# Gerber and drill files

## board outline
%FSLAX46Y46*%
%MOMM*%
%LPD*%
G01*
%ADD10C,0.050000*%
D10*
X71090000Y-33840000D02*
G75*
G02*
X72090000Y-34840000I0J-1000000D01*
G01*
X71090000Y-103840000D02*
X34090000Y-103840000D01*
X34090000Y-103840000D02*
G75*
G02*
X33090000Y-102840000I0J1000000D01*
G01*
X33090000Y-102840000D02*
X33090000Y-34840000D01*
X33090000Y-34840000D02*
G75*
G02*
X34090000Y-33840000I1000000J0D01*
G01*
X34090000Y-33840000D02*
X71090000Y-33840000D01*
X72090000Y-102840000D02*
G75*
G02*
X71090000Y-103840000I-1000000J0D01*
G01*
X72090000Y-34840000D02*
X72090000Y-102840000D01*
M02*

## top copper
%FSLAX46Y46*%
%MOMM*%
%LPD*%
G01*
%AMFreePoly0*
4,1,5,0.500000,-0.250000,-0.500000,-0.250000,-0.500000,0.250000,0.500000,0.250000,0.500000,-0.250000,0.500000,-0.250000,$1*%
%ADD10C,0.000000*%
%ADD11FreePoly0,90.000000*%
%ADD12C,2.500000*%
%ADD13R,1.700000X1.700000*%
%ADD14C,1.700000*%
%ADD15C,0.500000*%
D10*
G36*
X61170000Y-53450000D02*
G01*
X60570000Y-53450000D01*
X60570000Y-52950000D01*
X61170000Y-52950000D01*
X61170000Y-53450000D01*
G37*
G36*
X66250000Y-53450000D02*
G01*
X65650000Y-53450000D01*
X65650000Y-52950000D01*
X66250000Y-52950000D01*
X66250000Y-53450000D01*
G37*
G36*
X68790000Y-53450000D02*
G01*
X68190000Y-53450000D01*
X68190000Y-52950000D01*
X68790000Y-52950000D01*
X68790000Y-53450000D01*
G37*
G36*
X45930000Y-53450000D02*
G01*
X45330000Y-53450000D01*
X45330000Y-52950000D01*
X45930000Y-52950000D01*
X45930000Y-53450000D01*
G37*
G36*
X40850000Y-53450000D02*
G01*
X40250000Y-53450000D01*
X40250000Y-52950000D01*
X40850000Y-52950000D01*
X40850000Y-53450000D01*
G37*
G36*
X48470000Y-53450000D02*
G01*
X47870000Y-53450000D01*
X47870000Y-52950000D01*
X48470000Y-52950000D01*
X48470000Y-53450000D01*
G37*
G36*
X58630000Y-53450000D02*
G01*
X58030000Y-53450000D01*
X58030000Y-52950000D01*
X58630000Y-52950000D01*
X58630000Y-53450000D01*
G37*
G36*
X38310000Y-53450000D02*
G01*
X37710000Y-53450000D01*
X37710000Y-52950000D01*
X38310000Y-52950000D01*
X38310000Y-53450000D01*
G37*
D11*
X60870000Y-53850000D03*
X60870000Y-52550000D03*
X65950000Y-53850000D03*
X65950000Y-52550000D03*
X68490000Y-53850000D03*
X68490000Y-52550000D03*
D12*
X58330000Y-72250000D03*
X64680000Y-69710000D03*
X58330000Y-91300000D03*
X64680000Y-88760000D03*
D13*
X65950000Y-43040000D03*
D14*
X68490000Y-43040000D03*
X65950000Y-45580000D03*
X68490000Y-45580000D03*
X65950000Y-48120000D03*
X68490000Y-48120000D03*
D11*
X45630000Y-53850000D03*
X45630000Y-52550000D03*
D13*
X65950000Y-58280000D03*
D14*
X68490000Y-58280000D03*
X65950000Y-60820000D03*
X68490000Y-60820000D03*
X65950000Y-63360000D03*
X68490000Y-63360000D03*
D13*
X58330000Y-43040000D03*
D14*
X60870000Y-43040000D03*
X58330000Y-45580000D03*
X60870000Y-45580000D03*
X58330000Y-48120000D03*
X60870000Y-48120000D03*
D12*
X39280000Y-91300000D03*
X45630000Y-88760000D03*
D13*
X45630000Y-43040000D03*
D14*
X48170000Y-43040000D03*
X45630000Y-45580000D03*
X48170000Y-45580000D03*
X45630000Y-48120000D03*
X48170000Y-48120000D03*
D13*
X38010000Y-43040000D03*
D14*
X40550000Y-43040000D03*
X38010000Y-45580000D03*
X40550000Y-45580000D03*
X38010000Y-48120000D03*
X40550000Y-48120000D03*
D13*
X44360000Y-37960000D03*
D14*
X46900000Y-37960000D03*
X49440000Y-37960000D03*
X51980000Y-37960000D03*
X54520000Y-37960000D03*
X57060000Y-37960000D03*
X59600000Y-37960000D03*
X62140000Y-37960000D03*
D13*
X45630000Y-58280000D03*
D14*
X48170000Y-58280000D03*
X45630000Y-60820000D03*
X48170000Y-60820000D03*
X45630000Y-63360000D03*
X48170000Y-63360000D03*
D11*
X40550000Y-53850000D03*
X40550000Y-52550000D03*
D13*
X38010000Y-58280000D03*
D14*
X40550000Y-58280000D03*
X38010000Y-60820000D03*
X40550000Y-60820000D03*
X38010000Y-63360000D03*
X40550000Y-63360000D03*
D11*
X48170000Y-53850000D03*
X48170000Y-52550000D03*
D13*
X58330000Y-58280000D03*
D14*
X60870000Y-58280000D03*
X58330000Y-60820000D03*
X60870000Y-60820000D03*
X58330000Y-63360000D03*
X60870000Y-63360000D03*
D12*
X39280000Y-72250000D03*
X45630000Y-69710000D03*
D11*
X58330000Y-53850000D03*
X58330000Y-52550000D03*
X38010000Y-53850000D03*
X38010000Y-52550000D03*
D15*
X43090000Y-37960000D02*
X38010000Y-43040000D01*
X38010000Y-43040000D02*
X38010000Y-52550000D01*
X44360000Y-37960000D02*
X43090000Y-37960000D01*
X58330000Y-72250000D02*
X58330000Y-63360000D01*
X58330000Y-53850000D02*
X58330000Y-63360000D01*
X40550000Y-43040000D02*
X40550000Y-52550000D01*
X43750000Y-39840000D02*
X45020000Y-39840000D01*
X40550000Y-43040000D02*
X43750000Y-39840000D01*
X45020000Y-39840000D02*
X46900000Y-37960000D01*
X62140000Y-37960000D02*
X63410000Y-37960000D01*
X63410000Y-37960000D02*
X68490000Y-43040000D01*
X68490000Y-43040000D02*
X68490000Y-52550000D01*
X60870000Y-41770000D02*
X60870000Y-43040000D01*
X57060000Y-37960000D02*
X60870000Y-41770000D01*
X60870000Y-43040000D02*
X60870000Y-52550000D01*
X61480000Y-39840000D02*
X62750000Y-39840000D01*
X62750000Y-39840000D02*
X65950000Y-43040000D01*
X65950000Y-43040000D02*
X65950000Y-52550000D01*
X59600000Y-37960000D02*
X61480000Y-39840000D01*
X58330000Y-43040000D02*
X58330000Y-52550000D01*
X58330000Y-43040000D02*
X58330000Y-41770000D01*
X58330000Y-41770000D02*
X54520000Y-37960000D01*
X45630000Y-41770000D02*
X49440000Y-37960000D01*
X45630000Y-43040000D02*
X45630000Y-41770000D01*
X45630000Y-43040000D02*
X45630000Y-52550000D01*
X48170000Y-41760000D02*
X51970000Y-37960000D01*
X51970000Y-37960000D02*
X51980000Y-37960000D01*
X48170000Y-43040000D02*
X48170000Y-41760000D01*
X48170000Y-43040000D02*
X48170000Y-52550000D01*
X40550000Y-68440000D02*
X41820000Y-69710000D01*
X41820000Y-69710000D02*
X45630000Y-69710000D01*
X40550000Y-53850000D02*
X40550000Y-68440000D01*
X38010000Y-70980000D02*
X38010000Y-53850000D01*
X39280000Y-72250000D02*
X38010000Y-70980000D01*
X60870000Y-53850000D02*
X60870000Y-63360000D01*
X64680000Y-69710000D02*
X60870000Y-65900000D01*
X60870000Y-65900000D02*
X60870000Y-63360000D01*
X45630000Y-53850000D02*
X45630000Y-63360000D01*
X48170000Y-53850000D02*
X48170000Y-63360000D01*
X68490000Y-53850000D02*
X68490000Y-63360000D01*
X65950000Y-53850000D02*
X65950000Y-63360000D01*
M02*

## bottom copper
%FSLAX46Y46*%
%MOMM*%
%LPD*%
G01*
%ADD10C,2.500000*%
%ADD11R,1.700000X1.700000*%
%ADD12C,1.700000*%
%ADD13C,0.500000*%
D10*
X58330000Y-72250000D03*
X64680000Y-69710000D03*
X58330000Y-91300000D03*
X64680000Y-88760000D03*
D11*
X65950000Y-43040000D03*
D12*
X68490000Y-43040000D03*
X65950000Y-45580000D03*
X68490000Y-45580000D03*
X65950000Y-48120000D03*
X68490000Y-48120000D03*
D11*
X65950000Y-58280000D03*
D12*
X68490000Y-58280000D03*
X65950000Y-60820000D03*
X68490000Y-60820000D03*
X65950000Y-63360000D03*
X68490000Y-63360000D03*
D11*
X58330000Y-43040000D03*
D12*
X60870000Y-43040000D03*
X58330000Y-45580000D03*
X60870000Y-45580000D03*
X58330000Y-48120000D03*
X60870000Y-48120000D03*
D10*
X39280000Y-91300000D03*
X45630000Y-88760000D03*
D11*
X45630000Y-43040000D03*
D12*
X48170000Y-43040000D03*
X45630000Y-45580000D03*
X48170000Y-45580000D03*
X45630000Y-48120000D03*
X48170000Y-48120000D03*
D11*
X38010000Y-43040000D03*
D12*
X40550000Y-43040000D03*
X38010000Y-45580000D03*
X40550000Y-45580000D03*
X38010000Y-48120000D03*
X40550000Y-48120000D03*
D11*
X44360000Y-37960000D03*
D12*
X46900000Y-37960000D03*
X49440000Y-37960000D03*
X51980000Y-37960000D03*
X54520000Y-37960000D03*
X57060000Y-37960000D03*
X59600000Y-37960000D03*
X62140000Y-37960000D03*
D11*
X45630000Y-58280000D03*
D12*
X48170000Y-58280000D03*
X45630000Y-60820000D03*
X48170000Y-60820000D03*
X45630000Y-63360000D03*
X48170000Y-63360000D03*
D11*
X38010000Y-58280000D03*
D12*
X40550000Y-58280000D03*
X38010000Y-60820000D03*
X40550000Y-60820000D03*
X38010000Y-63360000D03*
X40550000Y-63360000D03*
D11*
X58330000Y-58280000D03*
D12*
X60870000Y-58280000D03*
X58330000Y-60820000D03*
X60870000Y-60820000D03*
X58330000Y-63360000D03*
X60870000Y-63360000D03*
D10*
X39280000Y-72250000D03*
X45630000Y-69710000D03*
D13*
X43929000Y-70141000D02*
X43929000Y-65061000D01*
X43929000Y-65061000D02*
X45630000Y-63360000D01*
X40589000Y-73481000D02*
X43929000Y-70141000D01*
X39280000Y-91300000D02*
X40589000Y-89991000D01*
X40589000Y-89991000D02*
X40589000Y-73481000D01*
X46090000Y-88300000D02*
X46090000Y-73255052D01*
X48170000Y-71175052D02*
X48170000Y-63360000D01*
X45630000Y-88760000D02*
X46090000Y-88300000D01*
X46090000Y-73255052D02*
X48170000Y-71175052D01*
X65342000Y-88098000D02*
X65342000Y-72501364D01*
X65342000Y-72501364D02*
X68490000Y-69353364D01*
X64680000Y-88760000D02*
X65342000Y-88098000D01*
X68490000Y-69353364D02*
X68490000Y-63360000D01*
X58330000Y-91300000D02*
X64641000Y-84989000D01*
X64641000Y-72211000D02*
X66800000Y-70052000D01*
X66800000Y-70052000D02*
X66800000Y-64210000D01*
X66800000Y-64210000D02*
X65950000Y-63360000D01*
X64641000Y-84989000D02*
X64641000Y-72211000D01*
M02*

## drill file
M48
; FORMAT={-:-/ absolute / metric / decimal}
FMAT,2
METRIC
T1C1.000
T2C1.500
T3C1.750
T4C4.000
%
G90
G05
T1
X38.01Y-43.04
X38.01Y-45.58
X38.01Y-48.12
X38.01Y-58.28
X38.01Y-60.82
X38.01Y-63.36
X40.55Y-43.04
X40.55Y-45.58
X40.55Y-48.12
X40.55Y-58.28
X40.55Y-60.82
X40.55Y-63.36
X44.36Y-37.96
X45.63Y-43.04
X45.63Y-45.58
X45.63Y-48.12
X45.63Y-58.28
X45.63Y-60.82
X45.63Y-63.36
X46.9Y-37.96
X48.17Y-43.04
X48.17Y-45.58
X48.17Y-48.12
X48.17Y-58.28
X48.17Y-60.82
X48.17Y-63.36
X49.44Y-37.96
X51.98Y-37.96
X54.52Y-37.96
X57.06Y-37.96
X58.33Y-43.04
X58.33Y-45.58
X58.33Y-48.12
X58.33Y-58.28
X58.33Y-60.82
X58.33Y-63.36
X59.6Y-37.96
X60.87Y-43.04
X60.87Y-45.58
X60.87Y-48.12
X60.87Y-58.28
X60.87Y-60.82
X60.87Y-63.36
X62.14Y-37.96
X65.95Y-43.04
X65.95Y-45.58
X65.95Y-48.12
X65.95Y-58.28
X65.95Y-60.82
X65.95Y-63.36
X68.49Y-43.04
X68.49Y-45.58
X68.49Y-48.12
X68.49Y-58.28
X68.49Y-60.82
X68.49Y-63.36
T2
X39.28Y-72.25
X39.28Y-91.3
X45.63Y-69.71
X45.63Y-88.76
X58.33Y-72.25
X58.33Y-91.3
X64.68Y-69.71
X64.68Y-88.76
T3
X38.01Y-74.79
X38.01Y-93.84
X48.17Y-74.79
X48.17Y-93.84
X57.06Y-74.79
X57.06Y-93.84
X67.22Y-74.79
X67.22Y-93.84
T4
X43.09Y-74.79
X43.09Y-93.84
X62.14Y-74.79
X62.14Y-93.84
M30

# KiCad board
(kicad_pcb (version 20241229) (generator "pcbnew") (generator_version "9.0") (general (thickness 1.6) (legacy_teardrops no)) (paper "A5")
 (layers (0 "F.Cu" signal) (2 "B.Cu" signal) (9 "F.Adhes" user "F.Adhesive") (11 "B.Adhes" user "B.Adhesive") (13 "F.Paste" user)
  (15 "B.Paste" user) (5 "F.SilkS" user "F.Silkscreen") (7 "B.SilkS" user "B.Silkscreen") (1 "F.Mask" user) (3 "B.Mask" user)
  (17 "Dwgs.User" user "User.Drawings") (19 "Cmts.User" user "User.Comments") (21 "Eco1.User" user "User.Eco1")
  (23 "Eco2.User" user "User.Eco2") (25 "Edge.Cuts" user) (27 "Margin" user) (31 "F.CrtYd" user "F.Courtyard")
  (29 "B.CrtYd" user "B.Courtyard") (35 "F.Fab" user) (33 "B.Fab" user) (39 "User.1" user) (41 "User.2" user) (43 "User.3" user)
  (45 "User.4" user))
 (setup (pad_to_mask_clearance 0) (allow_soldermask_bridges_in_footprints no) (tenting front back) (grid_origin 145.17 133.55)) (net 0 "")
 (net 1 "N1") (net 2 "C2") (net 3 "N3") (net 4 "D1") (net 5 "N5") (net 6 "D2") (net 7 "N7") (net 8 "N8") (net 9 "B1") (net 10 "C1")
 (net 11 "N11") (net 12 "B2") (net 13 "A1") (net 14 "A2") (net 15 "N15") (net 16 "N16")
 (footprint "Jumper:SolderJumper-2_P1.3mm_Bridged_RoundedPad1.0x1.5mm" (layer "F.Cu") (at 60.87 53.2 90)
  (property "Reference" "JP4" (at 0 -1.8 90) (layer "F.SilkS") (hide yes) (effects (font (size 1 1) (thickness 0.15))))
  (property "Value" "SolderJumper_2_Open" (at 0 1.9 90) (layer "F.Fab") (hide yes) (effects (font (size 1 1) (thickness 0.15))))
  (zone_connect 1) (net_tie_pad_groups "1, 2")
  (fp_poly (pts (xy 0.25 -0.3) (xy -0.25 -0.3) (xy -0.25 0.3) (xy 0.25 0.3)) (stroke (width 0) (type solid)) (fill yes) (layer "F.Cu"))
  (pad "1" smd custom (at -0.65 0 90) (size 1 0.5) (layers "F.Cu" "F.Mask") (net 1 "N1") (zone_connect 2) (thermal_bridge_angle 45)
   (options (clearance outline) (anchor rect)) (primitives))
  (pad "2" smd custom (at 0.65 0 90) (size 1 0.5) (layers "F.Cu" "F.Mask") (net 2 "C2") (zone_connect 2) (thermal_bridge_angle 45)
   (options (clearance outline) (anchor rect)) (primitives)))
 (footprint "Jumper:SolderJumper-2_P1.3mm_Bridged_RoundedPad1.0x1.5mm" (layer "F.Cu") (at 65.95 53.2 90)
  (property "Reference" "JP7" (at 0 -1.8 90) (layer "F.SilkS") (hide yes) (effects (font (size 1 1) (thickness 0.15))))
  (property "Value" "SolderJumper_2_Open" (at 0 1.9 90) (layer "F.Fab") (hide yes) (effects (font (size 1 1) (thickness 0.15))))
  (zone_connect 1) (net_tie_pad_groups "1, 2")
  (fp_poly (pts (xy 0.25 -0.3) (xy -0.25 -0.3) (xy -0.25 0.3) (xy 0.25 0.3)) (stroke (width 0) (type solid)) (fill yes) (layer "F.Cu"))
  (pad "1" smd custom (at -0.65 0 90) (size 1 0.5) (layers "F.Cu" "F.Mask") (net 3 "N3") (zone_connect 2) (thermal_bridge_angle 45)
   (options (clearance outline) (anchor rect)) (primitives))
  (pad "2" smd custom (at 0.65 0 90) (size 1 0.5) (layers "F.Cu" "F.Mask") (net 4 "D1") (zone_connect 2) (thermal_bridge_angle 45)
   (options (clearance outline) (anchor rect)) (primitives)))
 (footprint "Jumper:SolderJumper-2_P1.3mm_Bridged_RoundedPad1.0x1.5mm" (layer "F.Cu") (at 68.49 53.2 90)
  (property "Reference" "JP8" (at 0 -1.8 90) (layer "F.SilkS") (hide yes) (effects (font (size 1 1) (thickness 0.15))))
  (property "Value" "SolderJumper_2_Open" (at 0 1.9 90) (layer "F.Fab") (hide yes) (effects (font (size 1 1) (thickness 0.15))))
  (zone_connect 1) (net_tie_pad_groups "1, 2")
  (fp_poly (pts (xy 0.25 -0.3) (xy -0.25 -0.3) (xy -0.25 0.3) (xy 0.25 0.3)) (stroke (width 0) (type solid)) (fill yes) (layer "F.Cu"))
  (pad "1" smd custom (at -0.65 0 90) (size 1 0.5) (layers "F.Cu" "F.Mask") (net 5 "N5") (zone_connect 2) (thermal_bridge_angle 45)
   (options (clearance outline) (anchor rect)) (primitives))
  (pad "2" smd custom (at 0.65 0 90) (size 1 0.5) (layers "F.Cu" "F.Mask") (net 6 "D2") (zone_connect 2) (thermal_bridge_angle 45)
   (options (clearance outline) (anchor rect)) (primitives)))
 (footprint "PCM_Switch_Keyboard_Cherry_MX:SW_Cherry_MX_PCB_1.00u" (layer "F.Cu") (at 62.14 74.79)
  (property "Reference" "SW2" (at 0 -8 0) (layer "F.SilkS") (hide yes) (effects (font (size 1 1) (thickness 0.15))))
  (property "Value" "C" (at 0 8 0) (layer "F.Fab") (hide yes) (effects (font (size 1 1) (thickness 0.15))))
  (pad "" np_thru_hole circle (at -5.08 0) (size 1.75 1.75) (drill 1.75) (layers "*.Cu" "*.Mask"))
  (pad "" np_thru_hole circle (at 0 0) (size 4 4) (drill 4) (layers "*.Cu" "*.Mask"))
  (pad "" np_thru_hole circle (at 5.08 0) (size 1.75 1.75) (drill 1.75) (layers "*.Cu" "*.Mask"))
  (pad "1" thru_hole circle (at -3.81 -2.54) (size 2.5 2.5) (drill 1.5) (layers "*.Cu" "*.Mask") (remove_unused_layers no) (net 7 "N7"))
  (pad "2" thru_hole circle (at 2.54 -5.08) (size 2.5 2.5) (drill 1.5) (layers "*.Cu" "*.Mask") (remove_unused_layers no) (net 1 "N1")))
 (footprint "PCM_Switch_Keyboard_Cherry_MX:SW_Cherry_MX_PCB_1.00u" (layer "F.Cu") (at 62.14 93.84)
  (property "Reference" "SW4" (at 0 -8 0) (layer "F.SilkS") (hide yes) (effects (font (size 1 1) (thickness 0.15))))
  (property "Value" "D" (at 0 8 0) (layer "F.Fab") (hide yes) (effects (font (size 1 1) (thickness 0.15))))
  (pad "" np_thru_hole circle (at -5.08 0) (size 1.75 1.75) (drill 1.75) (layers "*.Cu" "*.Mask"))
  (pad "" np_thru_hole circle (at 0 0) (size 4 4) (drill 4) (layers "*.Cu" "*.Mask"))
  (pad "" np_thru_hole circle (at 5.08 0) (size 1.75 1.75) (drill 1.75) (layers "*.Cu" "*.Mask"))
  (pad "1" thru_hole circle (at -3.81 -2.54) (size 2.5 2.5) (drill 1.5) (layers "*.Cu" "*.Mask") (remove_unused_layers no) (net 3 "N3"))
  (pad "2" thru_hole circle (at 2.54 -5.08) (size 2.5 2.5) (drill 1.5) (layers "*.Cu" "*.Mask") (remove_unused_layers no) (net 5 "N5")))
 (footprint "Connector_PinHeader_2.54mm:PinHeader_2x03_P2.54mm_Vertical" (layer "F.Cu") (at 65.95 43.04)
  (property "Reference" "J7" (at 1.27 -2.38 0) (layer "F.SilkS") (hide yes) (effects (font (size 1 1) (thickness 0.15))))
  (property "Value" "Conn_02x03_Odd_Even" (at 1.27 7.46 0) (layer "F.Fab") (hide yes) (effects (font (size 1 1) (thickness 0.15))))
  (pad "1" thru_hole rect (at 0 0) (size 1.7 1.7) (drill 1) (layers "*.Cu" "*.Mask") (remove_unused_layers no) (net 4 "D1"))
  (pad "2" thru_hole circle (at 2.54 0) (size 1.7 1.7) (drill 1) (layers "*.Cu" "*.Mask") (remove_unused_layers no) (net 6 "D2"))
  (pad "3" thru_hole circle (at 0 2.54) (size 1.7 1.7) (drill 1) (layers "*.Cu" "*.Mask") (remove_unused_layers no) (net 4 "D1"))
  (pad "4" thru_hole circle (at 2.54 2.54) (size 1.7 1.7) (drill 1) (layers "*.Cu" "*.Mask") (remove_unused_layers no) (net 6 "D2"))
  (pad "5" thru_hole circle (at 0 5.08) (size 1.7 1.7) (drill 1) (layers "*.Cu" "*.Mask") (remove_unused_layers no) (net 4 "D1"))
  (pad "6" thru_hole circle (at 2.54 5.08) (size 1.7 1.7) (drill 1) (layers "*.Cu" "*.Mask") (remove_unused_layers no) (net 6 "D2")))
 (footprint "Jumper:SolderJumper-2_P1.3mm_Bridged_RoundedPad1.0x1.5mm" (layer "F.Cu") (at 45.63 53.2 90)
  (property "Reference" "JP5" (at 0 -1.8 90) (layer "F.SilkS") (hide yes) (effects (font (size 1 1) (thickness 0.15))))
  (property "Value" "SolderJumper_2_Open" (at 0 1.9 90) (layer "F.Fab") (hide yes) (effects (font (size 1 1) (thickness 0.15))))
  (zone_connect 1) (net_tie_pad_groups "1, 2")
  (fp_poly (pts (xy 0.25 -0.3) (xy -0.25 -0.3) (xy -0.25 0.3) (xy 0.25 0.3)) (stroke (width 0) (type solid)) (fill yes) (layer "F.Cu"))
  (pad "1" smd custom (at -0.65 0 90) (size 1 0.5) (layers "F.Cu" "F.Mask") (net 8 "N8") (zone_connect 2) (thermal_bridge_angle 45)
   (options (clearance outline) (anchor rect)) (primitives))
  (pad "2" smd custom (at 0.65 0 90) (size 1 0.5) (layers "F.Cu" "F.Mask") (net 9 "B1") (zone_connect 2) (thermal_bridge_angle 45)
   (options (clearance outline) (anchor rect)) (primitives)))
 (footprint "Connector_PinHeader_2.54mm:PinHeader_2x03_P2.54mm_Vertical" (layer "F.Cu") (at 65.95 58.28)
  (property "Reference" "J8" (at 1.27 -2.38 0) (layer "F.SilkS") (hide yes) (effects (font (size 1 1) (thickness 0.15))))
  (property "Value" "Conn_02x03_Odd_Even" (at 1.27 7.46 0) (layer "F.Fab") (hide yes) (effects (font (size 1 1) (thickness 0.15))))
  (pad "1" thru_hole rect (at 0 0) (size 1.7 1.7) (drill 1) (layers "*.Cu" "*.Mask") (remove_unused_layers no) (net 3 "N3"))
  (pad "2" thru_hole circle (at 2.54 0) (size 1.7 1.7) (drill 1) (layers "*.Cu" "*.Mask") (remove_unused_layers no) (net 5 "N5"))
  (pad "3" thru_hole circle (at 0 2.54) (size 1.7 1.7) (drill 1) (layers "*.Cu" "*.Mask") (remove_unused_layers no) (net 3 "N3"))
  (pad "4" thru_hole circle (at 2.54 2.54) (size 1.7 1.7) (drill 1) (layers "*.Cu" "*.Mask") (remove_unused_layers no) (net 5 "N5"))
  (pad "5" thru_hole circle (at 0 5.08) (size 1.7 1.7) (drill 1) (layers "*.Cu" "*.Mask") (remove_unused_layers no) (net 3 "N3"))
  (pad "6" thru_hole circle (at 2.54 5.08) (size 1.7 1.7) (drill 1) (layers "*.Cu" "*.Mask") (remove_unused_layers no) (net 5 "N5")))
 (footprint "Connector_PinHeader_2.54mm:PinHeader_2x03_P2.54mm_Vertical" (layer "F.Cu") (at 58.33 43.04)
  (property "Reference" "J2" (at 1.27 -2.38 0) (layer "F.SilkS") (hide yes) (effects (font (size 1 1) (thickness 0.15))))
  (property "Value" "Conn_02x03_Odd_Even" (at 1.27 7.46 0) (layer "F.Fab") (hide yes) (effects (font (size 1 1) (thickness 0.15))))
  (pad "1" thru_hole rect (at 0 0) (size 1.7 1.7) (drill 1) (layers "*.Cu" "*.Mask") (remove_unused_layers no) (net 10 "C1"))
  (pad "2" thru_hole circle (at 2.54 0) (size 1.7 1.7) (drill 1) (layers "*.Cu" "*.Mask") (remove_unused_layers no) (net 2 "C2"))
  (pad "3" thru_hole circle (at 0 2.54) (size 1.7 1.7) (drill 1) (layers "*.Cu" "*.Mask") (remove_unused_layers no) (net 10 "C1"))
  (pad "4" thru_hole circle (at 2.54 2.54) (size 1.7 1.7) (drill 1) (layers "*.Cu" "*.Mask") (remove_unused_layers no) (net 2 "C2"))
  (pad "5" thru_hole circle (at 0 5.08) (size 1.7 1.7) (drill 1) (layers "*.Cu" "*.Mask") (remove_unused_layers no) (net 10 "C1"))
  (pad "6" thru_hole circle (at 2.54 5.08) (size 1.7 1.7) (drill 1) (layers "*.Cu" "*.Mask") (remove_unused_layers no) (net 2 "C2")))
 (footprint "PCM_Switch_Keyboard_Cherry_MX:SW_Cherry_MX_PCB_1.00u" (layer "F.Cu") (at 43.09 93.84)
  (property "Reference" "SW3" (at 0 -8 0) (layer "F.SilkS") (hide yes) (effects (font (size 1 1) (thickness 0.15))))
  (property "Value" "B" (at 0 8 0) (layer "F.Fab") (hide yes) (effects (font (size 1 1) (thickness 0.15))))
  (pad "" np_thru_hole circle (at -5.08 0) (size 1.75 1.75) (drill 1.75) (layers "*.Cu" "*.Mask"))
  (pad "" np_thru_hole circle (at 0 0) (size 4 4) (drill 4) (layers "*.Cu" "*.Mask"))
  (pad "" np_thru_hole circle (at 5.08 0) (size 1.75 1.75) (drill 1.75) (layers "*.Cu" "*.Mask"))
  (pad "1" thru_hole circle (at -3.81 -2.54) (size 2.5 2.5) (drill 1.5) (layers "*.Cu" "*.Mask") (remove_unused_layers no) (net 8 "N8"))
  (pad "2" thru_hole circle (at 2.54 -5.08) (size 2.5 2.5) (drill 1.5) (layers "*.Cu" "*.Mask") (remove_unused_layers no) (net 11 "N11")))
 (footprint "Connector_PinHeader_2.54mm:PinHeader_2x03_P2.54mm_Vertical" (layer "F.Cu") (at 45.63 43.04)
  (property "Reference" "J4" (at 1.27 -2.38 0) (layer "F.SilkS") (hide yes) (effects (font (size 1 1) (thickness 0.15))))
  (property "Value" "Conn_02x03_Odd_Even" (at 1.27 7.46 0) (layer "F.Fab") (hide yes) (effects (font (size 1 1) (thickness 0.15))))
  (pad "1" thru_hole rect (at 0 0) (size 1.7 1.7) (drill 1) (layers "*.Cu" "*.Mask") (remove_unused_layers no) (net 9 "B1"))
  (pad "2" thru_hole circle (at 2.54 0) (size 1.7 1.7) (drill 1) (layers "*.Cu" "*.Mask") (remove_unused_layers no) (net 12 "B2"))
  (pad "3" thru_hole circle (at 0 2.54) (size 1.7 1.7) (drill 1) (layers "*.Cu" "*.Mask") (remove_unused_layers no) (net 9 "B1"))
  (pad "4" thru_hole circle (at 2.54 2.54) (size 1.7 1.7) (drill 1) (layers "*.Cu" "*.Mask") (remove_unused_layers no) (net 12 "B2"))
  (pad "5" thru_hole circle (at 0 5.08) (size 1.7 1.7) (drill 1) (layers "*.Cu" "*.Mask") (remove_unused_layers no) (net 9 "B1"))
  (pad "6" thru_hole circle (at 2.54 5.08) (size 1.7 1.7) (drill 1) (layers "*.Cu" "*.Mask") (remove_unused_layers no) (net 12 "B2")))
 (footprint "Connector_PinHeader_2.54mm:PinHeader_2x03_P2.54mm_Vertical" (layer "F.Cu") (at 38.01 43.04)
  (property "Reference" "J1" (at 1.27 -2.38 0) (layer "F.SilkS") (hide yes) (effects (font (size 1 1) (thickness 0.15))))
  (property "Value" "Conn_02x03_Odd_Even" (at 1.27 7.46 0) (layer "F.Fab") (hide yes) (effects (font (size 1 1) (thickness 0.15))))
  (pad "1" thru_hole rect (at 0 0) (size 1.7 1.7) (drill 1) (layers "*.Cu" "*.Mask") (remove_unused_layers no) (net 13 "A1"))
  (pad "2" thru_hole circle (at 2.54 0) (size 1.7 1.7) (drill 1) (layers "*.Cu" "*.Mask") (remove_unused_layers no) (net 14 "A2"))
  (pad "3" thru_hole circle (at 0 2.54) (size 1.7 1.7) (drill 1) (layers "*.Cu" "*.Mask") (remove_unused_layers no) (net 13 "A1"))
  (pad "4" thru_hole circle (at 2.54 2.54) (size 1.7 1.7) (drill 1) (layers "*.Cu" "*.Mask") (remove_unused_layers no) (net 14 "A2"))
  (pad "5" thru_hole circle (at 0 5.08) (size 1.7 1.7) (drill 1) (layers "*.Cu" "*.Mask") (remove_unused_layers no) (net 13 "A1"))
  (pad "6" thru_hole circle (at 2.54 5.08) (size 1.7 1.7) (drill 1) (layers "*.Cu" "*.Mask") (remove_unused_layers no) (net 14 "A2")))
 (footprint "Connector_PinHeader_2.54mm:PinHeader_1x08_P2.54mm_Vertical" (layer "F.Cu") (at 44.36 37.96 90)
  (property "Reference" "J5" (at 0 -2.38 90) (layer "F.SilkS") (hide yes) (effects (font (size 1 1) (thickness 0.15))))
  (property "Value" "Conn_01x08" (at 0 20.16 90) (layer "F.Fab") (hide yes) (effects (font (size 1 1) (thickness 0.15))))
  (pad "1" thru_hole rect (at 0 0 90) (size 1.7 1.7) (drill 1) (layers "*.Cu" "*.Mask") (remove_unused_layers no) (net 13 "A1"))
  (pad "2" thru_hole circle (at 0 2.54 90) (size 1.7 1.7) (drill 1) (layers "*.Cu" "*.Mask") (remove_unused_layers no) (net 14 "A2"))
  (pad "3" thru_hole circle (at 0 5.08 90) (size 1.7 1.7) (drill 1) (layers "*.Cu" "*.Mask") (remove_unused_layers no) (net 9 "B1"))
  (pad "4" thru_hole circle (at 0 7.62 90) (size 1.7 1.7) (drill 1) (layers "*.Cu" "*.Mask") (remove_unused_layers no) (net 12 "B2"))
  (pad "5" thru_hole circle (at 0 10.16 90) (size 1.7 1.7) (drill 1) (layers "*.Cu" "*.Mask") (remove_unused_layers no) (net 10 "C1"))
  (pad "6" thru_hole circle (at 0 12.7 90) (size 1.7 1.7) (drill 1) (layers "*.Cu" "*.Mask") (remove_unused_layers no) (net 2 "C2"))
  (pad "7" thru_hole circle (at 0 15.24 90) (size 1.7 1.7) (drill 1) (layers "*.Cu" "*.Mask") (remove_unused_layers no) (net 4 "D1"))
  (pad "8" thru_hole circle (at 0 17.78 90) (size 1.7 1.7) (drill 1) (layers "*.Cu" "*.Mask") (remove_unused_layers no) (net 6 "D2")))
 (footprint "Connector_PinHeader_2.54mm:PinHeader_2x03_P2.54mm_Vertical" (layer "F.Cu") (at 45.63 58.28)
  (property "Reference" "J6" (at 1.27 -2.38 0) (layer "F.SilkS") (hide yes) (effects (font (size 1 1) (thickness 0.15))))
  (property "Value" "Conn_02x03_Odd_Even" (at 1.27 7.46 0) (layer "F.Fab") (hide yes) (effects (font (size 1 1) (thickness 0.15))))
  (pad "1" thru_hole rect (at 0 0) (size 1.7 1.7) (drill 1) (layers "*.Cu" "*.Mask") (remove_unused_layers no) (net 8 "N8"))
  (pad "2" thru_hole circle (at 2.54 0) (size 1.7 1.7) (drill 1) (layers "*.Cu" "*.Mask") (remove_unused_layers no) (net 11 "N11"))
  (pad "3" thru_hole circle (at 0 2.54) (size 1.7 1.7) (drill 1) (layers "*.Cu" "*.Mask") (remove_unused_layers no) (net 8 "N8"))
  (pad "4" thru_hole circle (at 2.54 2.54) (size 1.7 1.7) (drill 1) (layers "*.Cu" "*.Mask") (remove_unused_layers no) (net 11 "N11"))
  (pad "5" thru_hole circle (at 0 5.08) (size 1.7 1.7) (drill 1) (layers "*.Cu" "*.Mask") (remove_unused_layers no) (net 8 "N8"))
  (pad "6" thru_hole circle (at 2.54 5.08) (size 1.7 1.7) (drill 1) (layers "*.Cu" "*.Mask") (remove_unused_layers no) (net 11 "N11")))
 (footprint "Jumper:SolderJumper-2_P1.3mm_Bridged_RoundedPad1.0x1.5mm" (layer "F.Cu") (at 40.55 53.2 90)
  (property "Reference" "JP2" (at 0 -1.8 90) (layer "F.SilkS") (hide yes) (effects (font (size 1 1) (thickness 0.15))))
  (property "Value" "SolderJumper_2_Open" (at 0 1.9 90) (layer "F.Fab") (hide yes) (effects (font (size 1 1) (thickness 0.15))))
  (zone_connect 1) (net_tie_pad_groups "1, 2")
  (fp_poly (pts (xy 0.25 -0.3) (xy -0.25 -0.3) (xy -0.25 0.3) (xy 0.25 0.3)) (stroke (width 0) (type solid)) (fill yes) (layer "F.Cu"))
  (pad "1" smd custom (at -0.65 0 90) (size 1 0.5) (layers "F.Cu" "F.Mask") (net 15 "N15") (zone_connect 2) (thermal_bridge_angle 45)
   (options (clearance outline) (anchor rect)) (primitives))
  (pad "2" smd custom (at 0.65 0 90) (size 1 0.5) (layers "F.Cu" "F.Mask") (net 14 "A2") (zone_connect 2) (thermal_bridge_angle 45)
   (options (clearance outline) (anchor rect)) (primitives)))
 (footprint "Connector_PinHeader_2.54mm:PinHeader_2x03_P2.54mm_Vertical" (layer "F.Cu") (at 38.01 58.28)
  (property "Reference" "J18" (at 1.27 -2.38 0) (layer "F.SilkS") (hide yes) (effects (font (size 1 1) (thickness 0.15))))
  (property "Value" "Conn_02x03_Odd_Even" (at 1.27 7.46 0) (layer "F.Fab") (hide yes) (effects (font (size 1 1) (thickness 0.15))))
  (pad "1" thru_hole rect (at 0 0) (size 1.7 1.7) (drill 1) (layers "*.Cu" "*.Mask") (remove_unused_layers no) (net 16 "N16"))
  (pad "2" thru_hole circle (at 2.54 0) (size 1.7 1.7) (drill 1) (layers "*.Cu" "*.Mask") (remove_unused_layers no) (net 15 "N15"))
  (pad "3" thru_hole circle (at 0 2.54) (size 1.7 1.7) (drill 1) (layers "*.Cu" "*.Mask") (remove_unused_layers no) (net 16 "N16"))
  (pad "4" thru_hole circle (at 2.54 2.54) (size 1.7 1.7) (drill 1) (layers "*.Cu" "*.Mask") (remove_unused_layers no) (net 15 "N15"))
  (pad "5" thru_hole circle (at 0 5.08) (size 1.7 1.7) (drill 1) (layers "*.Cu" "*.Mask") (remove_unused_layers no) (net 16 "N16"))
  (pad "6" thru_hole circle (at 2.54 5.08) (size 1.7 1.7) (drill 1) (layers "*.Cu" "*.Mask") (remove_unused_layers no) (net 15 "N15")))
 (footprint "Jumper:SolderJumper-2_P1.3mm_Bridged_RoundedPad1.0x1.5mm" (layer "F.Cu") (at 48.17 53.2 90)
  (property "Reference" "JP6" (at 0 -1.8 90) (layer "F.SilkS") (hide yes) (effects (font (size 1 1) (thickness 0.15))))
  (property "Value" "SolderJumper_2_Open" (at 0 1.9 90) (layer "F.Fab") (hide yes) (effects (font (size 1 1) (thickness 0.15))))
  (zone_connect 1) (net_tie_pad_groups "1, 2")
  (fp_poly (pts (xy 0.25 -0.3) (xy -0.25 -0.3) (xy -0.25 0.3) (xy 0.25 0.3)) (stroke (width 0) (type solid)) (fill yes) (layer "F.Cu"))
  (pad "1" smd custom (at -0.65 0 90) (size 1 0.5) (layers "F.Cu" "F.Mask") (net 11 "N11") (zone_connect 2) (thermal_bridge_angle 45)
   (options (clearance outline) (anchor rect)) (primitives))
  (pad "2" smd custom (at 0.65 0 90) (size 1 0.5) (layers "F.Cu" "F.Mask") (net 12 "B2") (zone_connect 2) (thermal_bridge_angle 45)
   (options (clearance outline) (anchor rect)) (primitives)))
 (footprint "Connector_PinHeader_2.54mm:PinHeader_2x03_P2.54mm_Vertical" (layer "F.Cu") (at 58.33 58.28)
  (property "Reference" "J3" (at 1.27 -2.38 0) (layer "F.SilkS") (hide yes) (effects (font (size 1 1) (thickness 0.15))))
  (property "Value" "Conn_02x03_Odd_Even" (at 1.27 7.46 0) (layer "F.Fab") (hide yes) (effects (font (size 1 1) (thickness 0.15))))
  (pad "1" thru_hole rect (at 0 0) (size 1.7 1.7) (drill 1) (layers "*.Cu" "*.Mask") (remove_unused_layers no) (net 7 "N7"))
  (pad "2" thru_hole circle (at 2.54 0) (size 1.7 1.7) (drill 1) (layers "*.Cu" "*.Mask") (remove_unused_layers no) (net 1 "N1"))
  (pad "3" thru_hole circle (at 0 2.54) (size 1.7 1.7) (drill 1) (layers "*.Cu" "*.Mask") (remove_unused_layers no) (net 7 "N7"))
  (pad "4" thru_hole circle (at 2.54 2.54) (size 1.7 1.7) (drill 1) (layers "*.Cu" "*.Mask") (remove_unused_layers no) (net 1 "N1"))
  (pad "5" thru_hole circle (at 0 5.08) (size 1.7 1.7) (drill 1) (layers "*.Cu" "*.Mask") (remove_unused_layers no) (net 7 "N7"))
  (pad "6" thru_hole circle (at 2.54 5.08) (size 1.7 1.7) (drill 1) (layers "*.Cu" "*.Mask") (remove_unused_layers no) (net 1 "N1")))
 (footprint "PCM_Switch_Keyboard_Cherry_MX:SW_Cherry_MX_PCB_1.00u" (layer "F.Cu") (at 43.09 74.79)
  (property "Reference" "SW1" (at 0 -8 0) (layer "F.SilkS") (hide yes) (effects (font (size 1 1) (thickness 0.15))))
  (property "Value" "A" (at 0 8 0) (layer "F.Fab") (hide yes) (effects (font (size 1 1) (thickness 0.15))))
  (pad "" np_thru_hole circle (at -5.08 0) (size 1.75 1.75) (drill 1.75) (layers "*.Cu" "*.Mask"))
  (pad "" np_thru_hole circle (at 0 0) (size 4 4) (drill 4) (layers "*.Cu" "*.Mask"))
  (pad "" np_thru_hole circle (at 5.08 0) (size 1.75 1.75) (drill 1.75) (layers "*.Cu" "*.Mask"))
  (pad "1" thru_hole circle (at -3.81 -2.54) (size 2.5 2.5) (drill 1.5) (layers "*.Cu" "*.Mask") (remove_unused_layers no) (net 16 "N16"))
  (pad "2" thru_hole circle (at 2.54 -5.08) (size 2.5 2.5) (drill 1.5) (layers "*.Cu" "*.Mask") (remove_unused_layers no) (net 15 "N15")))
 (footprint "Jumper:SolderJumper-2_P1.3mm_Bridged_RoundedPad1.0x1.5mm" (layer "F.Cu") (at 58.33 53.2 90)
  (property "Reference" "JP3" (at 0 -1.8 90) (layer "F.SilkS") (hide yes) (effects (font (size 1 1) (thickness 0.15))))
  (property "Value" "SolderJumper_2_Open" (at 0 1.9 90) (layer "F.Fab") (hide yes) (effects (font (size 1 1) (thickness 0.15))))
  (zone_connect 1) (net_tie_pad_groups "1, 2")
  (fp_poly (pts (xy 0.25 -0.3) (xy -0.25 -0.3) (xy -0.25 0.3) (xy 0.25 0.3)) (stroke (width 0) (type solid)) (fill yes) (layer "F.Cu"))
  (pad "1" smd custom (at -0.65 0 90) (size 1 0.5) (layers "F.Cu" "F.Mask") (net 7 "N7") (zone_connect 2) (thermal_bridge_angle 45)
   (options (clearance outline) (anchor rect)) (primitives))
  (pad "2" smd custom (at 0.65 0 90) (size 1 0.5) (layers "F.Cu" "F.Mask") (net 10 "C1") (zone_connect 2) (thermal_bridge_angle 45)
   (options (clearance outline) (anchor rect)) (primitives)))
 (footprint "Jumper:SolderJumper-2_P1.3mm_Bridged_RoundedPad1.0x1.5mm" (layer "F.Cu") (at 38.01 53.2 90)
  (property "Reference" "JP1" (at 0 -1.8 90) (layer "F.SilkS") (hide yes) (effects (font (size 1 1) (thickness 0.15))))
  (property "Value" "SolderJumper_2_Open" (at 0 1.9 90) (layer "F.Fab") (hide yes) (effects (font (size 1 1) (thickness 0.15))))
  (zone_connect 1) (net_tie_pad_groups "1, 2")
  (fp_poly (pts (xy 0.25 -0.3) (xy -0.25 -0.3) (xy -0.25 0.3) (xy 0.25 0.3)) (stroke (width 0) (type solid)) (fill yes) (layer "F.Cu"))
  (pad "1" smd custom (at -0.65 0 90) (size 1 0.5) (layers "F.Cu" "F.Mask") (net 16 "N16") (zone_connect 2) (thermal_bridge_angle 45)
   (options (clearance outline) (anchor rect)) (primitives))
  (pad "2" smd custom (at 0.65 0 90) (size 1 0.5) (layers "F.Cu" "F.Mask") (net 13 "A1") (zone_connect 2) (thermal_bridge_angle 45)
   (options (clearance outline) (anchor rect)) (primitives)))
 (gr_arc (start 71.09 33.84) (mid 71.797107 34.132893) (end 72.09 34.84) (stroke (width 0.05) (type default)) (layer "Edge.Cuts"))
 (gr_line (start 71.09 103.84) (end 34.09 103.84) (stroke (width 0.05) (type default)) (layer "Edge.Cuts"))
 (gr_arc (start 34.09 103.84) (mid 33.382893 103.547107) (end 33.09 102.84) (stroke (width 0.05) (type default)) (layer "Edge.Cuts"))
 (gr_line (start 33.09 102.84) (end 33.09 34.84) (stroke (width 0.05) (type default)) (layer "Edge.Cuts"))
 (gr_arc (start 33.09 34.84) (mid 33.382893 34.132893) (end 34.09 33.84) (stroke (width 0.05) (type default)) (layer "Edge.Cuts"))
 (gr_line (start 34.09 33.84) (end 71.09 33.84) (stroke (width 0.05) (type default)) (layer "Edge.Cuts"))
 (gr_arc (start 72.09 102.84) (mid 71.797107 103.547107) (end 71.09 103.84) (stroke (width 0.05) (type default)) (layer "Edge.Cuts"))
 (gr_line (start 72.09 34.84) (end 72.09 102.84) (stroke (width 0.05) (type default)) (layer "Edge.Cuts"))
 (segment (start 43.09 37.96) (end 38.01 43.04) (width 0.5) (layer "F.Cu") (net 13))
 (segment (start 38.01 43.04) (end 38.01 52.55) (width 0.5) (layer "F.Cu") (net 13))
 (segment (start 44.36 37.96) (end 43.09 37.96) (width 0.5) (layer "F.Cu") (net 13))
 (segment (start 58.33 72.25) (end 58.33 63.36) (width 0.5) (layer "F.Cu") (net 7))
 (segment (start 58.33 53.85) (end 58.33 63.36) (width 0.5) (layer "F.Cu") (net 7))
 (segment (start 40.55 43.04) (end 40.55 52.55) (width 0.5) (layer "F.Cu") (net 14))
 (segment (start 43.75 39.84) (end 45.02 39.84) (width 0.5) (layer "F.Cu") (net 14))
 (segment (start 40.55 43.04) (end 43.75 39.84) (width 0.5) (layer "F.Cu") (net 14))
 (segment (start 45.02 39.84) (end 46.9 37.96) (width 0.5) (layer "F.Cu") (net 14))
 (segment (start 62.14 37.96) (end 63.41 37.96) (width 0.5) (layer "F.Cu") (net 6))
 (segment (start 63.41 37.96) (end 68.49 43.04) (width 0.5) (layer "F.Cu") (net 6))
 (segment (start 68.49 43.04) (end 68.49 52.55) (width 0.5) (layer "F.Cu") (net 6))
 (segment (start 60.87 41.77) (end 60.87 43.04) (width 0.5) (layer "F.Cu") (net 2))
 (segment (start 57.06 37.96) (end 60.87 41.77) (width 0.5) (layer "F.Cu") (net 2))
 (segment (start 60.87 43.04) (end 60.87 52.55) (width 0.5) (layer "F.Cu") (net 2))
 (segment (start 61.48 39.84) (end 62.75 39.84) (width 0.5) (layer "F.Cu") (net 4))
 (segment (start 62.75 39.84) (end 65.95 43.04) (width 0.5) (layer "F.Cu") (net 4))
 (segment (start 65.95 43.04) (end 65.95 52.55) (width 0.5) (layer "F.Cu") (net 4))
 (segment (start 59.6 37.96) (end 61.48 39.84) (width 0.5) (layer "F.Cu") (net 4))
 (segment (start 58.33 43.04) (end 58.33 52.55) (width 0.5) (layer "F.Cu") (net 10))
 (segment (start 58.33 43.04) (end 58.33 41.77) (width 0.5) (layer "F.Cu") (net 10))
 (segment (start 58.33 41.77) (end 54.52 37.96) (width 0.5) (layer "F.Cu") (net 10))
 (segment (start 45.63 41.77) (end 49.44 37.96) (width 0.5) (layer "F.Cu") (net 9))
 (segment (start 45.63 43.04) (end 45.63 41.77) (width 0.5) (layer "F.Cu") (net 9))
 (segment (start 45.63 43.04) (end 45.63 52.55) (width 0.5) (layer "F.Cu") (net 9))
 (segment (start 48.17 41.76) (end 51.97 37.96) (width 0.5) (layer "F.Cu") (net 12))
 (segment (start 51.97 37.96) (end 51.98 37.96) (width 0.5) (layer "F.Cu") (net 12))
 (segment (start 48.17 43.04) (end 48.17 41.76) (width 0.5) (layer "F.Cu") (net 12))
 (segment (start 48.17 43.04) (end 48.17 52.55) (width 0.5) (layer "F.Cu") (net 12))
 (segment (start 40.55 68.44) (end 41.82 69.71) (width 0.5) (layer "F.Cu") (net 15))
 (segment (start 41.82 69.71) (end 45.63 69.71) (width 0.5) (layer "F.Cu") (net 15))
 (segment (start 40.55 53.85) (end 40.55 68.44) (width 0.5) (layer "F.Cu") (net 15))
 (segment (start 38.01 70.98) (end 38.01 53.85) (width 0.5) (layer "F.Cu") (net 16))
 (segment (start 39.28 72.25) (end 38.01 70.98) (width 0.5) (layer "F.Cu") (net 16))
 (segment (start 60.87 53.85) (end 60.87 63.36) (width 0.5) (layer "F.Cu") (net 1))
 (segment (start 64.68 69.71) (end 60.87 65.9) (width 0.5) (layer "F.Cu") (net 1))
 (segment (start 60.87 65.9) (end 60.87 63.36) (width 0.5) (layer "F.Cu") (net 1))
 (segment (start 45.63 53.85) (end 45.63 63.36) (width 0.5) (layer "F.Cu") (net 8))
 (segment (start 43.929 70.141) (end 43.929 65.061) (width 0.5) (layer "B.Cu") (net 8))
 (segment (start 43.929 65.061) (end 45.63 63.36) (width 0.5) (layer "B.Cu") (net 8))
 (segment (start 40.589 73.481) (end 43.929 70.141) (width 0.5) (layer "B.Cu") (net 8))
 (segment (start 39.28 91.3) (end 40.589 89.991) (width 0.5) (layer "B.Cu") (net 8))
 (segment (start 40.589 89.991) (end 40.589 73.481) (width 0.5) (layer "B.Cu") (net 8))
 (segment (start 48.17 53.85) (end 48.17 63.36) (width 0.5) (layer "F.Cu") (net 11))
 (segment (start 46.09 88.3) (end 46.09 73.255052) (width 0.5) (layer "B.Cu") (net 11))
 (segment (start 48.17 71.175052) (end 48.17 63.36) (width 0.5) (layer "B.Cu") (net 11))
 (segment (start 45.63 88.76) (end 46.09 88.3) (width 0.5) (layer "B.Cu") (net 11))
 (segment (start 46.09 73.255052) (end 48.17 71.175052) (width 0.5) (layer "B.Cu") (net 11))
 (segment (start 68.49 53.85) (end 68.49 63.36) (width 0.5) (layer "F.Cu") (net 5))
 (segment (start 65.342 88.098) (end 65.342 72.501364) (width 0.5) (layer "B.Cu") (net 5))
 (segment (start 65.342 72.501364) (end 68.49 69.353364) (width 0.5) (layer "B.Cu") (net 5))
 (segment (start 64.68 88.76) (end 65.342 88.098) (width 0.5) (layer "B.Cu") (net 5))
 (segment (start 68.49 69.353364) (end 68.49 63.36) (width 0.5) (layer "B.Cu") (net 5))
 (segment (start 65.95 53.85) (end 65.95 63.36) (width 0.5) (layer "F.Cu") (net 3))
 (segment (start 58.33 91.3) (end 64.641 84.989) (width 0.5) (layer "B.Cu") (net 3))
 (segment (start 64.641 72.211) (end 66.8 70.052) (width 0.5) (layer "B.Cu") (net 3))
 (segment (start 66.8 70.052) (end 66.8 64.21) (width 0.5) (layer "B.Cu") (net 3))
 (segment (start 66.8 64.21) (end 65.95 63.36) (width 0.5) (layer "B.Cu") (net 3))
 (segment (start 64.641 84.989) (end 64.641 72.211) (width 0.5) (layer "B.Cu") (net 3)))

